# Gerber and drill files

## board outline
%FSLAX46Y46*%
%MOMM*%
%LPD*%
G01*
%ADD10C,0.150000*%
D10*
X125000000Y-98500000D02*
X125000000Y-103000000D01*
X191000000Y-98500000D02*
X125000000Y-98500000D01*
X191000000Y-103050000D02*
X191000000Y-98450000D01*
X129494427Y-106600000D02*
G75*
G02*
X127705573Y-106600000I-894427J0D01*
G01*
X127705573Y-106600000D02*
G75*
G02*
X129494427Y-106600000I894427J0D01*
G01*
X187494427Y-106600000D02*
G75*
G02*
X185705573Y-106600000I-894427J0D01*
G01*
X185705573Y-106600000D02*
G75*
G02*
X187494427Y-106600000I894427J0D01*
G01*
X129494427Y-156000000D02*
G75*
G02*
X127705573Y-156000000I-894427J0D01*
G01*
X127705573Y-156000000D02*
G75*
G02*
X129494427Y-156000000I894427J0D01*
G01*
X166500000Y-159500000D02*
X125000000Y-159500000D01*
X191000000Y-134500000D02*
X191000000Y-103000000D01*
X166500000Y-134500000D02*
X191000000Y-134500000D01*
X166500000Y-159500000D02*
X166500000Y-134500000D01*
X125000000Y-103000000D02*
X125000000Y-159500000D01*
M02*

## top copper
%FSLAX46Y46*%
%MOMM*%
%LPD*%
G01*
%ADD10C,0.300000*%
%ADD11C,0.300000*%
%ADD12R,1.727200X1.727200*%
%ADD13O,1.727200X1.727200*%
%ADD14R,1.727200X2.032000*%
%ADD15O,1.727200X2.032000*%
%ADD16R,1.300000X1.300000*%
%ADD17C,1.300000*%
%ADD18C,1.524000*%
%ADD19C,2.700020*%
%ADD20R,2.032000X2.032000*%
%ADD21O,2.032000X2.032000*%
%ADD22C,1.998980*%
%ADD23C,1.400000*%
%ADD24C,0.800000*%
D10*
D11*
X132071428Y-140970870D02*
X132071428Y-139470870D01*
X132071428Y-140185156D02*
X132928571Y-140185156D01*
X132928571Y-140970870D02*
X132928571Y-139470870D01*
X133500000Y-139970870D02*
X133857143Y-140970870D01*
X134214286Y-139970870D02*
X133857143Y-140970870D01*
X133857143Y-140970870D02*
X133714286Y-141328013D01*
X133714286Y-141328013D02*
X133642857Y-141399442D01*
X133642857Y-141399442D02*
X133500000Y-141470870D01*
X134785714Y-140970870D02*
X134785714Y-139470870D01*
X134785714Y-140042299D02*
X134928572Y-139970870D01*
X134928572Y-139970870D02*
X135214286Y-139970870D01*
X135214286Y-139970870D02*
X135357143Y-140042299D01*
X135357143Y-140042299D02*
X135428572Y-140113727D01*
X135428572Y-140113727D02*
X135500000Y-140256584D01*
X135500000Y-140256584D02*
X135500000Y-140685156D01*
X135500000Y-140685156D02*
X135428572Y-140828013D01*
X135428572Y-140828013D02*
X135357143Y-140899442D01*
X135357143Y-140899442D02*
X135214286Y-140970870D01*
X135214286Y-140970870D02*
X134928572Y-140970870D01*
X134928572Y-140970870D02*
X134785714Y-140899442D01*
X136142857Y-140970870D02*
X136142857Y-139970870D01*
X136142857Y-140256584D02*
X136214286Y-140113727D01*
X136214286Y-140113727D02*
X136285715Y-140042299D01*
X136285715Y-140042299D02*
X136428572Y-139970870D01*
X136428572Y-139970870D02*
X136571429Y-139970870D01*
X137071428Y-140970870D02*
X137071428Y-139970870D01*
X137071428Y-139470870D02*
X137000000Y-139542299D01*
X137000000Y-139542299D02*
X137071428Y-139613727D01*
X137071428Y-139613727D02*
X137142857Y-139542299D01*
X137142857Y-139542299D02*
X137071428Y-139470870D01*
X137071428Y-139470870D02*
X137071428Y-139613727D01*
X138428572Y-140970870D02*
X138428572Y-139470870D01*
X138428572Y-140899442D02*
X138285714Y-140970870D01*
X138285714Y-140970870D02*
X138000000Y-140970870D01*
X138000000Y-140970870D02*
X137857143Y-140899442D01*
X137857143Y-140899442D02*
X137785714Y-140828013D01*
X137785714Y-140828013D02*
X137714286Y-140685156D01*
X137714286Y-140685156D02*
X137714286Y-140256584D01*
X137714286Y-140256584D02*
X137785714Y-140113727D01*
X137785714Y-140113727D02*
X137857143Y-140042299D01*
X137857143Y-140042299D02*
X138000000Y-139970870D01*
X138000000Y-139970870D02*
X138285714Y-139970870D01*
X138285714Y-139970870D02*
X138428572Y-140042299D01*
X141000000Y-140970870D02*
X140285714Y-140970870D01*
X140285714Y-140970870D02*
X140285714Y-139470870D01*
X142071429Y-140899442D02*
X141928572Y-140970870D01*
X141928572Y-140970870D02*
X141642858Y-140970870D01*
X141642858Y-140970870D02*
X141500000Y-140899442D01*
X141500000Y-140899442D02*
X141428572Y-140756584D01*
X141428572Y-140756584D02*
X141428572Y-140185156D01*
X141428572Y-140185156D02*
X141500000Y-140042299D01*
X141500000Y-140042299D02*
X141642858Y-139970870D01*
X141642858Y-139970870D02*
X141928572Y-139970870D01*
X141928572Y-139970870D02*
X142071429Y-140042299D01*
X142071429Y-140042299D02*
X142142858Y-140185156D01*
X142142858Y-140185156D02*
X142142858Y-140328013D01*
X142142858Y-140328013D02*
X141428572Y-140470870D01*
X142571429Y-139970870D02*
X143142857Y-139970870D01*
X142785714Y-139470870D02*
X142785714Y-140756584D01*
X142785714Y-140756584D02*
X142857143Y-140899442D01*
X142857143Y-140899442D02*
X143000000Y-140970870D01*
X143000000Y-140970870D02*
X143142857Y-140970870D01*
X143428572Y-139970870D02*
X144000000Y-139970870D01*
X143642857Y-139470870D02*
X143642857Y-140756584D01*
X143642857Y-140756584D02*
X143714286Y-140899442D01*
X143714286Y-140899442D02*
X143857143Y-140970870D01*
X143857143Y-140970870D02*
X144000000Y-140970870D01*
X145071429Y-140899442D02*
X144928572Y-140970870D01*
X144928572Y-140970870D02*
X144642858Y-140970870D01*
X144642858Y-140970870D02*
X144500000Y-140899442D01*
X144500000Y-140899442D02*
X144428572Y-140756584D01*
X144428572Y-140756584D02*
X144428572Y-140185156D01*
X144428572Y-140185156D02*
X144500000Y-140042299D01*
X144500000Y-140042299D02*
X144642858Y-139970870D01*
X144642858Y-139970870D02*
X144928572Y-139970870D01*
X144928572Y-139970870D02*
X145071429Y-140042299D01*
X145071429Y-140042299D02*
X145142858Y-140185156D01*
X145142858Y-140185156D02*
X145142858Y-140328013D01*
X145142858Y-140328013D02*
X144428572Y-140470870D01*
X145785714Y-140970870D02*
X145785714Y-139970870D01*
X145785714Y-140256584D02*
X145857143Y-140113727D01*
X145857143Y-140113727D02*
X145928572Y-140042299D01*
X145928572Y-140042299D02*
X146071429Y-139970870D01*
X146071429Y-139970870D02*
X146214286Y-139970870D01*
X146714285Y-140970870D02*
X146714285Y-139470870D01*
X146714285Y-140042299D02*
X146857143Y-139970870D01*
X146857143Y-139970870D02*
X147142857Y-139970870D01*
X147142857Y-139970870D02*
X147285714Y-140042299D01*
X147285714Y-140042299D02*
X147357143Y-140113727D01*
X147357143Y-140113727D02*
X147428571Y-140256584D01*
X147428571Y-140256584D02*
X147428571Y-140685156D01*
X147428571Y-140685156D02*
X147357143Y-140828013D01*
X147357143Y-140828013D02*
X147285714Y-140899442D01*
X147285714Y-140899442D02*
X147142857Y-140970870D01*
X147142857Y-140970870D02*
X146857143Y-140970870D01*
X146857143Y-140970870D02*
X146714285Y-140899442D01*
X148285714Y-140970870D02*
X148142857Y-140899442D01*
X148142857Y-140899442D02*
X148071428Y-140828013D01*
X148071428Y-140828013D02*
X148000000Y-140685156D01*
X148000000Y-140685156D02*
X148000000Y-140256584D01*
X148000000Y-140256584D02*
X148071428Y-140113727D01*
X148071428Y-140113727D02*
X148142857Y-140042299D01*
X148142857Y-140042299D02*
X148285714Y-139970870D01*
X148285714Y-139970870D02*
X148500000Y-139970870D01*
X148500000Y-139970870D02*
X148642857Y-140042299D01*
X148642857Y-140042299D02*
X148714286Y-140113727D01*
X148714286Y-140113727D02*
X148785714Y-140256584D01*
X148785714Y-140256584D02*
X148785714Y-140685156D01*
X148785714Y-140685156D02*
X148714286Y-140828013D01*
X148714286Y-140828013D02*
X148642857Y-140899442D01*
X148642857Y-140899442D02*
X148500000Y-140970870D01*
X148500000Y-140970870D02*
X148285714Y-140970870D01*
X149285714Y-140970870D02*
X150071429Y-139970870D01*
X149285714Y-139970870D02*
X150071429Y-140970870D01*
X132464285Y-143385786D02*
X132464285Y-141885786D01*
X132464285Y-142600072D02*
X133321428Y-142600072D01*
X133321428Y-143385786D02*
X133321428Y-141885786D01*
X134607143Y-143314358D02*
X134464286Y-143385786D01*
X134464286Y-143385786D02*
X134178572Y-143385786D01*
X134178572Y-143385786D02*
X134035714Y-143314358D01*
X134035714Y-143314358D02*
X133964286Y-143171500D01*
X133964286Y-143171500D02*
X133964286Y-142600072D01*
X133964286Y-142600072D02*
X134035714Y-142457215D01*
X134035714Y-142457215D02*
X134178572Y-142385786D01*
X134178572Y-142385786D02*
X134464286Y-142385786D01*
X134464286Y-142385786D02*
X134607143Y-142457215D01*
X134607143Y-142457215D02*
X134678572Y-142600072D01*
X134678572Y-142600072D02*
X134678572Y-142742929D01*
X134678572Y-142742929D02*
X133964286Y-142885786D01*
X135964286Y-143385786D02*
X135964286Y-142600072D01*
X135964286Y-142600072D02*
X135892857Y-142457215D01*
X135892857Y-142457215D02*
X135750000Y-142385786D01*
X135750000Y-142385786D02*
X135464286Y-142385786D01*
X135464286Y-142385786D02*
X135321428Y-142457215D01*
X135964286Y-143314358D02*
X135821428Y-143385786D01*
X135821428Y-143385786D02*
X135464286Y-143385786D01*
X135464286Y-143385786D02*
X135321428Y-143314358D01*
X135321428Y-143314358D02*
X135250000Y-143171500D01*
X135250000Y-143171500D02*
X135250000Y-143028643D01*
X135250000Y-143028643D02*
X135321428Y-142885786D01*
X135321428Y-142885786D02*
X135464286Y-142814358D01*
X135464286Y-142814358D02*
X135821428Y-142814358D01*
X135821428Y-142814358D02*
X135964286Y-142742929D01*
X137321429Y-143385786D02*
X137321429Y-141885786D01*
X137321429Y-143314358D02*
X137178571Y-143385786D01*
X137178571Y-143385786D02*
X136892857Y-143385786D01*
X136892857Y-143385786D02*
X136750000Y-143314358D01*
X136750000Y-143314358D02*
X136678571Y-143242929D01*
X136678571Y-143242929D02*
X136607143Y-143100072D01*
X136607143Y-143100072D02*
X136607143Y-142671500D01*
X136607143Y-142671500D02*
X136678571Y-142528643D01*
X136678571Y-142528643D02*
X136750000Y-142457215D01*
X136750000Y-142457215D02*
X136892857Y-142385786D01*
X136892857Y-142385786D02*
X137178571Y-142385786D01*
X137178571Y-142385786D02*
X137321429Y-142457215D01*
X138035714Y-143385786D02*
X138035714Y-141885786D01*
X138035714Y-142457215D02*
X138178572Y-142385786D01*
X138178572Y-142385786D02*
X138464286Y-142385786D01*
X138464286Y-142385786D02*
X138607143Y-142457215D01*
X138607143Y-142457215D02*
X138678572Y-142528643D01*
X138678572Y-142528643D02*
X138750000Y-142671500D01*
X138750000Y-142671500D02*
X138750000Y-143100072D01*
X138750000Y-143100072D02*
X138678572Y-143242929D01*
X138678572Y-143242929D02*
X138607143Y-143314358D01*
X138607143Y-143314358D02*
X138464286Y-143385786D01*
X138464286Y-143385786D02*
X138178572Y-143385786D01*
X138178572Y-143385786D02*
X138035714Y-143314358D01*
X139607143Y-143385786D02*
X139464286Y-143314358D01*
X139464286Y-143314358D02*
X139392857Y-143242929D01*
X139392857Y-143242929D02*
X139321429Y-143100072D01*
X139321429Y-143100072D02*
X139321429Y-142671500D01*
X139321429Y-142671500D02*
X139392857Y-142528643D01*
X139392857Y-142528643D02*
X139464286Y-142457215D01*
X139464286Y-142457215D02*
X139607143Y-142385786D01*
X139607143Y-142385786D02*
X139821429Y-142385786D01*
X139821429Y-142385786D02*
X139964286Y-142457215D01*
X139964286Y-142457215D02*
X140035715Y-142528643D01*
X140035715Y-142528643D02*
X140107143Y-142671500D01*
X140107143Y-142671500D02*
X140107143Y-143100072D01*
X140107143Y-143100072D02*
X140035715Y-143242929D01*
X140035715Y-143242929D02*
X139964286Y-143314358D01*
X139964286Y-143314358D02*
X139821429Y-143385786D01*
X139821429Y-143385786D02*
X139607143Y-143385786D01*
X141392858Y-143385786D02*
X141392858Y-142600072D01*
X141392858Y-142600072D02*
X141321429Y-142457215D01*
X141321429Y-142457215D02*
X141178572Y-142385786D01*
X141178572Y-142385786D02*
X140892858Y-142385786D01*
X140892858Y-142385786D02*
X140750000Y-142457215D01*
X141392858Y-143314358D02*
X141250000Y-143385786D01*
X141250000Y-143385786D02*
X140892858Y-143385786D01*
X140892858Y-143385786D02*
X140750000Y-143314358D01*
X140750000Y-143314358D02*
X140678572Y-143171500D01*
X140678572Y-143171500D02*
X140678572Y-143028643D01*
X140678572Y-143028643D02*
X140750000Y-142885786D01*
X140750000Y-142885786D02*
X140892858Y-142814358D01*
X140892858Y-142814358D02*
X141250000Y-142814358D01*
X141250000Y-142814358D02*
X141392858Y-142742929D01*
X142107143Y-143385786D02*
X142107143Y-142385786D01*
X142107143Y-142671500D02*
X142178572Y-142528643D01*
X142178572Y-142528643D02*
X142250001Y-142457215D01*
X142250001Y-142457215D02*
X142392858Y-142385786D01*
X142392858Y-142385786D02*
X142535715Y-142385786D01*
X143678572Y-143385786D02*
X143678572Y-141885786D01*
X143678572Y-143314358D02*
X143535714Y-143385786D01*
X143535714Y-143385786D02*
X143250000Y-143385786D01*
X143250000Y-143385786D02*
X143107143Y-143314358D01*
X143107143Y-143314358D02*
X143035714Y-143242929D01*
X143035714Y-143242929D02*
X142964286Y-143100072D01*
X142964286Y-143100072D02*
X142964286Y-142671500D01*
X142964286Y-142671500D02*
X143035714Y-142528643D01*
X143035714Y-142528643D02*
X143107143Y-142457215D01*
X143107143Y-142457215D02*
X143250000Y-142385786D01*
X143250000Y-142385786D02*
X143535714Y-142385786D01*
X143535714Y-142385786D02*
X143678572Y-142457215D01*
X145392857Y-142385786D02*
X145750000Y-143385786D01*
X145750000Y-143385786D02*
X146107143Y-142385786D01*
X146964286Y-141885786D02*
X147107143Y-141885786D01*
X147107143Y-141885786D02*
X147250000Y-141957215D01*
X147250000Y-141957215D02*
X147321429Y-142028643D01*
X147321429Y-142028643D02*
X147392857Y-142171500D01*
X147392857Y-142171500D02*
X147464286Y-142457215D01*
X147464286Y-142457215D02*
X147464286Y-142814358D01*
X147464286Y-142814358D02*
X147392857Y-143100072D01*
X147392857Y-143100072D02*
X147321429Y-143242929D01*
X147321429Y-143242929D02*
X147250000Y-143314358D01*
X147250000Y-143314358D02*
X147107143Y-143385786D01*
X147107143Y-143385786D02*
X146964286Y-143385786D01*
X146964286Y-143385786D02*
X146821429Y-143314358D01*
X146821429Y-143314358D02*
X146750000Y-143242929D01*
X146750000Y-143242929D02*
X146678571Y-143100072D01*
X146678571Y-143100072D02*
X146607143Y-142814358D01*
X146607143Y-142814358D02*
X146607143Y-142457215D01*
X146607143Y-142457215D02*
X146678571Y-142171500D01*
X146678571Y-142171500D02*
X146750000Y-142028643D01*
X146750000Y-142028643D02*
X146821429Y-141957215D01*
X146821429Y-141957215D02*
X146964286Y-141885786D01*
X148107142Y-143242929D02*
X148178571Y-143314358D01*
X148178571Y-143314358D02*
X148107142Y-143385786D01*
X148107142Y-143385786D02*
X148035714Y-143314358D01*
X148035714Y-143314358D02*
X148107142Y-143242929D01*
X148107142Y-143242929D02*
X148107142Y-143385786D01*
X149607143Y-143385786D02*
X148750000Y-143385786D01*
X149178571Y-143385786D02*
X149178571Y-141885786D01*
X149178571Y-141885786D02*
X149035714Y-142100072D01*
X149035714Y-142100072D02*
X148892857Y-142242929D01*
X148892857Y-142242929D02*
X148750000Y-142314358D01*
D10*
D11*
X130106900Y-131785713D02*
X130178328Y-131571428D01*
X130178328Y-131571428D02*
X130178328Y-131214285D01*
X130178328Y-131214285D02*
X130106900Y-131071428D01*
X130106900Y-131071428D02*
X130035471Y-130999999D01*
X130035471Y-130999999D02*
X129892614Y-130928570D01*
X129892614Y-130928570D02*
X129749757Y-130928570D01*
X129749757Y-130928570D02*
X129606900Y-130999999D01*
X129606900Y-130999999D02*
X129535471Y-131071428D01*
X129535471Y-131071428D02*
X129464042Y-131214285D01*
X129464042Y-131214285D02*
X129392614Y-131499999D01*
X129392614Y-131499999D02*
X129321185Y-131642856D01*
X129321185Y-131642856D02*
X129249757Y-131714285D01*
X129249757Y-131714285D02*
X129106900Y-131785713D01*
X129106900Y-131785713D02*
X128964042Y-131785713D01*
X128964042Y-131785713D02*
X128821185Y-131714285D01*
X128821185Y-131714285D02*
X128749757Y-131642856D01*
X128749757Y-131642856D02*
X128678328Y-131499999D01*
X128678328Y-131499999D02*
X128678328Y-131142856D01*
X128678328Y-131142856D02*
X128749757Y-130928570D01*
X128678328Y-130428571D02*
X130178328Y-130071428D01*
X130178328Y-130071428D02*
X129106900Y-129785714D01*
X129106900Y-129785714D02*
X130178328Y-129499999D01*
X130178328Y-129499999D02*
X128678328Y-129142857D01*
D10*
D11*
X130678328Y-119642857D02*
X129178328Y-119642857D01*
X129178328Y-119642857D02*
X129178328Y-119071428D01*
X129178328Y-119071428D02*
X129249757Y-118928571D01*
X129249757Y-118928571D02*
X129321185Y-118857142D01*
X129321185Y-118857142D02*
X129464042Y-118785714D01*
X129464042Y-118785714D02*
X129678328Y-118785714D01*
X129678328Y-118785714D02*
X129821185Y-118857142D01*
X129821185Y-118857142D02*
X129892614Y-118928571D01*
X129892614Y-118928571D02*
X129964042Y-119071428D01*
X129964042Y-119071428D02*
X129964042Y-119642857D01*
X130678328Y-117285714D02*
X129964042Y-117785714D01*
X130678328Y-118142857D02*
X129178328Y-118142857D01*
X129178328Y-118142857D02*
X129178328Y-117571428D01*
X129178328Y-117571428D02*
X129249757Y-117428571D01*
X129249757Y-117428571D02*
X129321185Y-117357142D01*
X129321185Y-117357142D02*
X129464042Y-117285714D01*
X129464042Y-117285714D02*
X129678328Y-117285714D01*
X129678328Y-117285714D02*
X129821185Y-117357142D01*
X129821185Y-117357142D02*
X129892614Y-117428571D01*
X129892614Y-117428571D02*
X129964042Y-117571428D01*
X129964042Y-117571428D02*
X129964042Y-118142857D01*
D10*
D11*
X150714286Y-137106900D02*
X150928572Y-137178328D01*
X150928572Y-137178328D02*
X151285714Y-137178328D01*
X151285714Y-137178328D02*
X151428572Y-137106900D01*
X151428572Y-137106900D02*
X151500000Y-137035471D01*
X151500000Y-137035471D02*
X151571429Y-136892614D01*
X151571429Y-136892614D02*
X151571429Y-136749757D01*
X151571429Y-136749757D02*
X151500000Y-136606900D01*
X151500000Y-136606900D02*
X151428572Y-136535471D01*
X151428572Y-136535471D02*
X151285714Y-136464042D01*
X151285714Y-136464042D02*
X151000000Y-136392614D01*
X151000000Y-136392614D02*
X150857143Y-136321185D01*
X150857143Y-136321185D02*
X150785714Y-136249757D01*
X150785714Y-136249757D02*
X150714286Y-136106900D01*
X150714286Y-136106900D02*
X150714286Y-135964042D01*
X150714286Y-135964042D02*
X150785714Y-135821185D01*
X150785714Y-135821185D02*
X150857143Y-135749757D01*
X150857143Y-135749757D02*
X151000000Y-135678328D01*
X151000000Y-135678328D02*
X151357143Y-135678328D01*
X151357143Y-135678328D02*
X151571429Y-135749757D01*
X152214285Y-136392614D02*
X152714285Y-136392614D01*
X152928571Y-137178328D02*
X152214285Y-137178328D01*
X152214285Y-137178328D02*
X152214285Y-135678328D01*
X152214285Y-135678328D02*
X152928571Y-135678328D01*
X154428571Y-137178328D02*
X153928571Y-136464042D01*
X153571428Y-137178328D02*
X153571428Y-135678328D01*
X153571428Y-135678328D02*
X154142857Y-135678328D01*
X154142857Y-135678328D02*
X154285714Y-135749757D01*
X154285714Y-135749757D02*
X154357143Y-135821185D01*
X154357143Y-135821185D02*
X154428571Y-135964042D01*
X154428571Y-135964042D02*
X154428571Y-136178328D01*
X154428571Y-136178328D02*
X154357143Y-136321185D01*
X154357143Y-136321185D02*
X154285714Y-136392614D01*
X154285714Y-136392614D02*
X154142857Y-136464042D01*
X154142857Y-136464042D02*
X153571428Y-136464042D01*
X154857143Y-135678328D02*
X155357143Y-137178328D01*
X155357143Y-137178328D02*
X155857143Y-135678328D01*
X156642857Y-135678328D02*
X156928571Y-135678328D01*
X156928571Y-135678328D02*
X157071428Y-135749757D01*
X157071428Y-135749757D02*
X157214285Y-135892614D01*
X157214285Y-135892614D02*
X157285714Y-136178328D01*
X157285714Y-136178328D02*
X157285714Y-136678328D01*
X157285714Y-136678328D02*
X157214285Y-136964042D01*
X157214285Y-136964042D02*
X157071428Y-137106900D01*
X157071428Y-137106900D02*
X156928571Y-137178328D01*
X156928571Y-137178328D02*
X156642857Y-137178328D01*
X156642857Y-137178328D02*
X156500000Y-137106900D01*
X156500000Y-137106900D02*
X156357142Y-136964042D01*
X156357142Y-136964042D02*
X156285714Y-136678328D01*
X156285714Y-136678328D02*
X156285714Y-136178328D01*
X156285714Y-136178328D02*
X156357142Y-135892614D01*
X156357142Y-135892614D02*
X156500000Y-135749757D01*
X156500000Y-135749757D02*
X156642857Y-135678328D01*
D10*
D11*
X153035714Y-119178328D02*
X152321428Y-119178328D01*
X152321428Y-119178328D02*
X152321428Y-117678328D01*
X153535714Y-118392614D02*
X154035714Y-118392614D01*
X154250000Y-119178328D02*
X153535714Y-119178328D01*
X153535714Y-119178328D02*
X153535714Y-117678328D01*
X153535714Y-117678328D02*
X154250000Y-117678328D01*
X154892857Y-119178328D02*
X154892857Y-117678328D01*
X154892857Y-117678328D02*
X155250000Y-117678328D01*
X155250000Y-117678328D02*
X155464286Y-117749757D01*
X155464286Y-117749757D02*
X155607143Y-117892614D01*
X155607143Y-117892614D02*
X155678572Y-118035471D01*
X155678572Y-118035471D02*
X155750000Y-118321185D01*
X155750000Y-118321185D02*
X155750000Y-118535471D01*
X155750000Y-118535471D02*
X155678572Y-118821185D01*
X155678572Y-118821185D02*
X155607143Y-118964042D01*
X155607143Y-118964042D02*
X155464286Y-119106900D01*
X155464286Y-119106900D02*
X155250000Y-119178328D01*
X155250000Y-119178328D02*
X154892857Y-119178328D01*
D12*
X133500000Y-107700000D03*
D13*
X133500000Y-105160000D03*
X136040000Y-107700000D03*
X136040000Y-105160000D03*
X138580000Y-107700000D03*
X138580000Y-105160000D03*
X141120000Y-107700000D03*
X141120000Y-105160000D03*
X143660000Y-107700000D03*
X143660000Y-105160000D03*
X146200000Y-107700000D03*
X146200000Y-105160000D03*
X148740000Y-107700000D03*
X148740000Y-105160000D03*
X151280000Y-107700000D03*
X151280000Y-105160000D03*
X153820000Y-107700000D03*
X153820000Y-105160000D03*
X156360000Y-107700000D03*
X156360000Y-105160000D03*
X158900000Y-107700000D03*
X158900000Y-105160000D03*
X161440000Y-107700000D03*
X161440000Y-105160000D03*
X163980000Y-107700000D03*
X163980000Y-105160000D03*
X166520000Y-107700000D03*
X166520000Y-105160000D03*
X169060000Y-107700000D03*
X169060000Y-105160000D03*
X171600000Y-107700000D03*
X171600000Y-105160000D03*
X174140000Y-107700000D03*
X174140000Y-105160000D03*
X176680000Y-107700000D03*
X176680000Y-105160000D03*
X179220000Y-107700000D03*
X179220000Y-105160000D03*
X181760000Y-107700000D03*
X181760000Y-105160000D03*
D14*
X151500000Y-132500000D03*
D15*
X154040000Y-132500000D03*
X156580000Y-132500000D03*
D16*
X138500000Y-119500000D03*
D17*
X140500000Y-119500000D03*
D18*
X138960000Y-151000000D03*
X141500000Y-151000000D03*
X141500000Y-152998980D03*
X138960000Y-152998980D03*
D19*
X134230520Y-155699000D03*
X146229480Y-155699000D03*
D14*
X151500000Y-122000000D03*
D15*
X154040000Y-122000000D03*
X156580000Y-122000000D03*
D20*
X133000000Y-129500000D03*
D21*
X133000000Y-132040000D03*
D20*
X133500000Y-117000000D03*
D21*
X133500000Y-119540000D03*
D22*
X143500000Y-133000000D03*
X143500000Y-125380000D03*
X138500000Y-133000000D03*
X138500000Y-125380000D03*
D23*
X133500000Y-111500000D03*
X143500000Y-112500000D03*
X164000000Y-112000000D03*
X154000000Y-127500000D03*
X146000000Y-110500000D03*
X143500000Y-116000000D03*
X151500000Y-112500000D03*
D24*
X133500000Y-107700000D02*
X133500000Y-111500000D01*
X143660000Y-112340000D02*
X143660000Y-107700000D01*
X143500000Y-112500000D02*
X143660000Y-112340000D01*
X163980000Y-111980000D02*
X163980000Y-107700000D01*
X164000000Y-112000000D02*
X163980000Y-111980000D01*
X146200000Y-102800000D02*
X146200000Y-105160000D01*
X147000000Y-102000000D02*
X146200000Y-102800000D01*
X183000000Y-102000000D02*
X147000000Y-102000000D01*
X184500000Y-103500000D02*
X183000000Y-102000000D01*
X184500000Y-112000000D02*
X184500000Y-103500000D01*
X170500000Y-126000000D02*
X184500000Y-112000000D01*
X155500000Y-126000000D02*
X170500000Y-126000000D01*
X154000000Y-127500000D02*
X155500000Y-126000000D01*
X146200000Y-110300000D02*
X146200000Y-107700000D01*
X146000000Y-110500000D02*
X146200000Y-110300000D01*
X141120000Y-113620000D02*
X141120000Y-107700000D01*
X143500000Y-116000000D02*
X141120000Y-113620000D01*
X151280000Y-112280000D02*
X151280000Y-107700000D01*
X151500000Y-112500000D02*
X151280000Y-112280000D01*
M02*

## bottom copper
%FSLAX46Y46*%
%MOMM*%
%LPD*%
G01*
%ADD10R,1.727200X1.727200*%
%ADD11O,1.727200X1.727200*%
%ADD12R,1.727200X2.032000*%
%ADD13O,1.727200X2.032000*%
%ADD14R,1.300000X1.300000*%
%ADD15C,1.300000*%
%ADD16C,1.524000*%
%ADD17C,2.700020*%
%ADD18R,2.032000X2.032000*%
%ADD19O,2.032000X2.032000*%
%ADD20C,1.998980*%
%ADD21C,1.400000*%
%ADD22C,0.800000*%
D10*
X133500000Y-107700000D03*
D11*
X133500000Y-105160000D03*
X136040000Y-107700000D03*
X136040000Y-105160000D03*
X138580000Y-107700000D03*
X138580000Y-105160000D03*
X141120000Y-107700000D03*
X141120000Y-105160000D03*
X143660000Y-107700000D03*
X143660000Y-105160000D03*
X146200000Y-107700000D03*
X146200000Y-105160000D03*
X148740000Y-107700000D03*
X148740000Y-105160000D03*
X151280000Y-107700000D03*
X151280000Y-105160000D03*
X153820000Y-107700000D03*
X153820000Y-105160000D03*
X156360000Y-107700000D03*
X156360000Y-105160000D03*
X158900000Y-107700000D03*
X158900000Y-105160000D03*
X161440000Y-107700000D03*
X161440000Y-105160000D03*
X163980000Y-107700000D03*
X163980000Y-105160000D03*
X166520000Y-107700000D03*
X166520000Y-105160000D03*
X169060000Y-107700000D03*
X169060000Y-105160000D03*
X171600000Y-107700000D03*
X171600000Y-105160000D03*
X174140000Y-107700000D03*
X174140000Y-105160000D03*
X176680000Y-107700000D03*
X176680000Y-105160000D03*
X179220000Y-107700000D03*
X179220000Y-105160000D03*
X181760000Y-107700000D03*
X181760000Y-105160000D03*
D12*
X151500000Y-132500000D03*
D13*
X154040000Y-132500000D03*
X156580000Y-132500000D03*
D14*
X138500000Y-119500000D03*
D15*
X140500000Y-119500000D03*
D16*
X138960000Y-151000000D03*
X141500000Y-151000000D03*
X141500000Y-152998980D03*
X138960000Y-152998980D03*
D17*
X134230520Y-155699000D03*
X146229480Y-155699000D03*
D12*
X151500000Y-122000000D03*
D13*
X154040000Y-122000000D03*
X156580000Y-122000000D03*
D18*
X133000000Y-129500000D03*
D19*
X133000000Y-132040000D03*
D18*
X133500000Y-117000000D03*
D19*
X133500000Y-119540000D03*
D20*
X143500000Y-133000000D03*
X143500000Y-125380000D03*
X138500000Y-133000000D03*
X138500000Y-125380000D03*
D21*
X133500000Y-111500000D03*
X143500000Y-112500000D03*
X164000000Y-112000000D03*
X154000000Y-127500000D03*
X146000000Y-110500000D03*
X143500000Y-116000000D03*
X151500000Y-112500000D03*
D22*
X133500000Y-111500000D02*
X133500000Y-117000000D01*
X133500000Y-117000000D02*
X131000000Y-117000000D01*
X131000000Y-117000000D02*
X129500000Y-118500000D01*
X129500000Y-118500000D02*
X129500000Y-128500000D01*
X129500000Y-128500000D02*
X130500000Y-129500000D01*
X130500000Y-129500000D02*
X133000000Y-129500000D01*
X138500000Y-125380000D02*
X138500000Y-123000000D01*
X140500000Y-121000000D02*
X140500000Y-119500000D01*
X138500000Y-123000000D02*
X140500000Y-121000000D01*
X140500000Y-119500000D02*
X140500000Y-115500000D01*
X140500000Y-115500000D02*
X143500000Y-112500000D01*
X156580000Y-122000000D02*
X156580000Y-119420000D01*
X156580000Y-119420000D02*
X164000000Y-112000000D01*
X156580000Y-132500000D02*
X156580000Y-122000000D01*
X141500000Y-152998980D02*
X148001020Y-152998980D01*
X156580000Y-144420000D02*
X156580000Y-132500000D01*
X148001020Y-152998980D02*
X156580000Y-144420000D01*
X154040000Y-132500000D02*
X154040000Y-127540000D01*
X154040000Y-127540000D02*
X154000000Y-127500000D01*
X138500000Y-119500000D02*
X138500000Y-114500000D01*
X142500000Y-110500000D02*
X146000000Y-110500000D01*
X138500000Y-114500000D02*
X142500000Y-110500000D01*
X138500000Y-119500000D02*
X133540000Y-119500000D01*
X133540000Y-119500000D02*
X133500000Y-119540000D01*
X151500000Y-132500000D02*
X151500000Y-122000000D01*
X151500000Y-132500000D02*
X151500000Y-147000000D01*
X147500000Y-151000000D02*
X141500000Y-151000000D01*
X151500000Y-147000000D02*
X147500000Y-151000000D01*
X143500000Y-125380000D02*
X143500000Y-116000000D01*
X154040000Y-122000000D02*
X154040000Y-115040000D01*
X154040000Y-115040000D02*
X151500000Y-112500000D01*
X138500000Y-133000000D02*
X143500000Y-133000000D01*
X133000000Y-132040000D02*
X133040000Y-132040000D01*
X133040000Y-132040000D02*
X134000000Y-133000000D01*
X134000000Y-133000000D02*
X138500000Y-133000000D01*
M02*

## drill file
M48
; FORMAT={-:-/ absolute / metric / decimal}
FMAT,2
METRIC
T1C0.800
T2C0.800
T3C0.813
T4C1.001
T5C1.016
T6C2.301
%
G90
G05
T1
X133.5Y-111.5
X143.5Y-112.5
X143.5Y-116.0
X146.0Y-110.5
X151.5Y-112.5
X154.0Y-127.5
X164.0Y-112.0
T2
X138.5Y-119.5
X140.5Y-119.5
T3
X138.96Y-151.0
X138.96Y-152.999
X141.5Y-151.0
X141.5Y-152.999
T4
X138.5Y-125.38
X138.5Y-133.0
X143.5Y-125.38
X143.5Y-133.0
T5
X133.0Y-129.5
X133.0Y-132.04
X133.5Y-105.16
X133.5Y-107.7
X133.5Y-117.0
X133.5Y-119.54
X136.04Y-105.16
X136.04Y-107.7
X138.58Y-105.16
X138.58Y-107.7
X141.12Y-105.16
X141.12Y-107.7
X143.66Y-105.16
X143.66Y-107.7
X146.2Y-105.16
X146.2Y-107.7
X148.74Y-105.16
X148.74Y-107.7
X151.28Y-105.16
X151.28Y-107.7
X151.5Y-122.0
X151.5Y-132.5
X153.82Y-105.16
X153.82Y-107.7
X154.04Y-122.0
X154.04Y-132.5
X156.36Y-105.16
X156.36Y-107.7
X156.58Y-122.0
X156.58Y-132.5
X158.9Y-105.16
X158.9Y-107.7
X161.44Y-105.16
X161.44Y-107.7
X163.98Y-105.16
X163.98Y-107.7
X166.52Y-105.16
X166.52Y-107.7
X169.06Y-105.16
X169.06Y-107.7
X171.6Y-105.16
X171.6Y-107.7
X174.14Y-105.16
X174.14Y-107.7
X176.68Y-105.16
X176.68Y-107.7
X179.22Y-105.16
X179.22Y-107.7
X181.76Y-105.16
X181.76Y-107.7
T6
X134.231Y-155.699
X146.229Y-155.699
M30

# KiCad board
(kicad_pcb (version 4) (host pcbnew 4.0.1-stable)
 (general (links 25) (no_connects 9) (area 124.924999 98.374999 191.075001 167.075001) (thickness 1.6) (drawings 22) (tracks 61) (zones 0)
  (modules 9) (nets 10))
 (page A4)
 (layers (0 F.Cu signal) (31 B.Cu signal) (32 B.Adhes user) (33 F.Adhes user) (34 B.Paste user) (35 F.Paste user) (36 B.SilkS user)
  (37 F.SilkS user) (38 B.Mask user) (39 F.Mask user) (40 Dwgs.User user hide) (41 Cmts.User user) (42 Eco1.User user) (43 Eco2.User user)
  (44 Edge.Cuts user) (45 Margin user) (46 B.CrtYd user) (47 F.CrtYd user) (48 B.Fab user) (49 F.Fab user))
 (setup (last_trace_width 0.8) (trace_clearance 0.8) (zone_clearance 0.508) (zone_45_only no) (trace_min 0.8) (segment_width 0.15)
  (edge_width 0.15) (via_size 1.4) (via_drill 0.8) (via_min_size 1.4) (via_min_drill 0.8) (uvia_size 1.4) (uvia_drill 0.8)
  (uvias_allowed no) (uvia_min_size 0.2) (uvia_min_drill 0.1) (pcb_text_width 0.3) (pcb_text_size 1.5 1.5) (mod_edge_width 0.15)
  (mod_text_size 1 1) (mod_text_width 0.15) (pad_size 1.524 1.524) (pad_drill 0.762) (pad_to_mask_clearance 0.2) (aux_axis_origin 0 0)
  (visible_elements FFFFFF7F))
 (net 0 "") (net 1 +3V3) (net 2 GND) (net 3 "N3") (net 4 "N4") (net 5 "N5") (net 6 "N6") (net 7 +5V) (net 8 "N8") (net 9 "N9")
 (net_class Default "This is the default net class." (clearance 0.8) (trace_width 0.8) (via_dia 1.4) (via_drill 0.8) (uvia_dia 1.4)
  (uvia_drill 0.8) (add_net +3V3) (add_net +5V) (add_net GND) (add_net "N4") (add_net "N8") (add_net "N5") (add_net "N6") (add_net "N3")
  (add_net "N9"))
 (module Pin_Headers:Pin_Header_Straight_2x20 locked (layer F.Cu) (at 133.5 107.7 90)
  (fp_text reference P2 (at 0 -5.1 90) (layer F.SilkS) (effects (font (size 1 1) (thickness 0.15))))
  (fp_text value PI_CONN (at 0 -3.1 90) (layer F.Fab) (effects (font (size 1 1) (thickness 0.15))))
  (pad 1 thru_hole rect (at 0 0 90) (size 1.7272 1.7272) (drill 1.016) (layers *.Cu *.Mask F.SilkS) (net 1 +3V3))
  (pad 2 thru_hole oval (at 2.54 0 90) (size 1.7272 1.7272) (drill 1.016) (layers *.Cu *.Mask F.SilkS))
  (pad 3 thru_hole oval (at 0 2.54 90) (size 1.7272 1.7272) (drill 1.016) (layers *.Cu *.Mask F.SilkS))
  (pad 4 thru_hole oval (at 2.54 2.54 90) (size 1.7272 1.7272) (drill 1.016) (layers *.Cu *.Mask F.SilkS))
  (pad 5 thru_hole oval (at 0 5.08 90) (size 1.7272 1.7272) (drill 1.016) (layers *.Cu *.Mask F.SilkS))
  (pad 6 thru_hole oval (at 2.54 5.08 90) (size 1.7272 1.7272) (drill 1.016) (layers *.Cu *.Mask F.SilkS) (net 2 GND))
  (pad 7 thru_hole oval (at 0 7.62 90) (size 1.7272 1.7272) (drill 1.016) (layers *.Cu *.Mask F.SilkS) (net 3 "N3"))
  (pad 8 thru_hole oval (at 2.54 7.62 90) (size 1.7272 1.7272) (drill 1.016) (layers *.Cu *.Mask F.SilkS))
  (pad 9 thru_hole oval (at 0 10.16 90) (size 1.7272 1.7272) (drill 1.016) (layers *.Cu *.Mask F.SilkS) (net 2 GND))
  (pad 10 thru_hole oval (at 2.54 10.16 90) (size 1.7272 1.7272) (drill 1.016) (layers *.Cu *.Mask F.SilkS))
  (pad 11 thru_hole oval (at 0 12.7 90) (size 1.7272 1.7272) (drill 1.016) (layers *.Cu *.Mask F.SilkS) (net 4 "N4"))
  (pad 12 thru_hole oval (at 2.54 12.7 90) (size 1.7272 1.7272) (drill 1.016) (layers *.Cu *.Mask F.SilkS) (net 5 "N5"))
  (pad 13 thru_hole oval (at 0 15.24 90) (size 1.7272 1.7272) (drill 1.016) (layers *.Cu *.Mask F.SilkS))
  (pad 14 thru_hole oval (at 2.54 15.24 90) (size 1.7272 1.7272) (drill 1.016) (layers *.Cu *.Mask F.SilkS) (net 2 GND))
  (pad 15 thru_hole oval (at 0 17.78 90) (size 1.7272 1.7272) (drill 1.016) (layers *.Cu *.Mask F.SilkS) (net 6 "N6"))
  (pad 16 thru_hole oval (at 2.54 17.78 90) (size 1.7272 1.7272) (drill 1.016) (layers *.Cu *.Mask F.SilkS))
  (pad 17 thru_hole oval (at 0 20.32 90) (size 1.7272 1.7272) (drill 1.016) (layers *.Cu *.Mask F.SilkS) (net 1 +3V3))
  (pad 18 thru_hole oval (at 2.54 20.32 90) (size 1.7272 1.7272) (drill 1.016) (layers *.Cu *.Mask F.SilkS))
  (pad 19 thru_hole oval (at 0 22.86 90) (size 1.7272 1.7272) (drill 1.016) (layers *.Cu *.Mask F.SilkS))
  (pad 20 thru_hole oval (at 2.54 22.86 90) (size 1.7272 1.7272) (drill 1.016) (layers *.Cu *.Mask F.SilkS) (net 2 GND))
  (pad 21 thru_hole oval (at 0 25.4 90) (size 1.7272 1.7272) (drill 1.016) (layers *.Cu *.Mask F.SilkS))
  (pad 22 thru_hole oval (at 2.54 25.4 90) (size 1.7272 1.7272) (drill 1.016) (layers *.Cu *.Mask F.SilkS))
  (pad 23 thru_hole oval (at 0 27.94 90) (size 1.7272 1.7272) (drill 1.016) (layers *.Cu *.Mask F.SilkS))
  (pad 24 thru_hole oval (at 2.54 27.94 90) (size 1.7272 1.7272) (drill 1.016) (layers *.Cu *.Mask F.SilkS))
  (pad 25 thru_hole oval (at 0 30.48 90) (size 1.7272 1.7272) (drill 1.016) (layers *.Cu *.Mask F.SilkS) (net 2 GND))
  (pad 26 thru_hole oval (at 2.54 30.48 90) (size 1.7272 1.7272) (drill 1.016) (layers *.Cu *.Mask F.SilkS))
  (pad 27 thru_hole oval (at 0 33.02 90) (size 1.7272 1.7272) (drill 1.016) (layers *.Cu *.Mask F.SilkS))
  (pad 28 thru_hole oval (at 2.54 33.02 90) (size 1.7272 1.7272) (drill 1.016) (layers *.Cu *.Mask F.SilkS))
  (pad 29 thru_hole oval (at 0 35.56 90) (size 1.7272 1.7272) (drill 1.016) (layers *.Cu *.Mask F.SilkS))
  (pad 30 thru_hole oval (at 2.54 35.56 90) (size 1.7272 1.7272) (drill 1.016) (layers *.Cu *.Mask F.SilkS) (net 2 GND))
  (pad 31 thru_hole oval (at 0 38.1 90) (size 1.7272 1.7272) (drill 1.016) (layers *.Cu *.Mask F.SilkS))
  (pad 32 thru_hole oval (at 2.54 38.1 90) (size 1.7272 1.7272) (drill 1.016) (layers *.Cu *.Mask F.SilkS))
  (pad 33 thru_hole oval (at 0 40.64 90) (size 1.7272 1.7272) (drill 1.016) (layers *.Cu *.Mask F.SilkS))
  (pad 34 thru_hole oval (at 2.54 40.64 90) (size 1.7272 1.7272) (drill 1.016) (layers *.Cu *.Mask F.SilkS) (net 2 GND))
  (pad 35 thru_hole oval (at 0 43.18 90) (size 1.7272 1.7272) (drill 1.016) (layers *.Cu *.Mask F.SilkS))
  (pad 36 thru_hole oval (at 2.54 43.18 90) (size 1.7272 1.7272) (drill 1.016) (layers *.Cu *.Mask F.SilkS))
  (pad 37 thru_hole oval (at 0 45.72 90) (size 1.7272 1.7272) (drill 1.016) (layers *.Cu *.Mask F.SilkS))
  (pad 38 thru_hole oval (at 2.54 45.72 90) (size 1.7272 1.7272) (drill 1.016) (layers *.Cu *.Mask F.SilkS))
  (pad 39 thru_hole oval (at 0 48.26 90) (size 1.7272 1.7272) (drill 1.016) (layers *.Cu *.Mask F.SilkS) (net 2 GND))
  (pad 40 thru_hole oval (at 2.54 48.26 90) (size 1.7272 1.7272) (drill 1.016) (layers *.Cu *.Mask F.SilkS)))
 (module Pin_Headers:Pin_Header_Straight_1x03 (layer F.Cu) (at 151.5 132.5 90)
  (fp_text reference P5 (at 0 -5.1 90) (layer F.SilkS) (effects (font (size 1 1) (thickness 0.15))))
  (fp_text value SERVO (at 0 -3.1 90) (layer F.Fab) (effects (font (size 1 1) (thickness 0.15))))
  (pad 1 thru_hole rect (at 0 0 90) (size 2.032 1.7272) (drill 1.016) (layers *.Cu *.Mask F.SilkS) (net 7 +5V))
  (pad 2 thru_hole oval (at 0 2.54 90) (size 2.032 1.7272) (drill 1.016) (layers *.Cu *.Mask F.SilkS) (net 5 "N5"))
  (pad 3 thru_hole oval (at 0 5.08 90) (size 2.032 1.7272) (drill 1.016) (layers *.Cu *.Mask F.SilkS) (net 2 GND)))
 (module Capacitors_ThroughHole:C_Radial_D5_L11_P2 (layer F.Cu) (at 138.5 119.5)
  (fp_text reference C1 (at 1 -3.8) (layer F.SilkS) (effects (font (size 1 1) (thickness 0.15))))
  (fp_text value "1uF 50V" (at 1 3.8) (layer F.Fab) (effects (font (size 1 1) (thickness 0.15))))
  (pad 1 thru_hole rect (at 0 0) (size 1.3 1.3) (drill 0.8) (layers *.Cu *.Mask F.SilkS) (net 4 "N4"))
  (pad 2 thru_hole circle (at 2 0) (size 1.3 1.3) (drill 0.8) (layers *.Cu *.Mask F.SilkS) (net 2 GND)))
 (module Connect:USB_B (layer F.Cu) (at 141.5 151 270)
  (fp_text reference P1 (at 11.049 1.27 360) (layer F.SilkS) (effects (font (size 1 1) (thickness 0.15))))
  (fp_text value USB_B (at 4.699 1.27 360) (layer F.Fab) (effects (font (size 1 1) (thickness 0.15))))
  (pad 2 thru_hole circle (at 0 2.54 180) (size 1.524 1.524) (drill 0.8128) (layers *.Cu *.Mask F.SilkS))
  (pad 1 thru_hole circle (at 0 0 180) (size 1.524 1.524) (drill 0.8128) (layers *.Cu *.Mask F.SilkS) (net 7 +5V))
  (pad 4 thru_hole circle (at 1.99898 0 180) (size 1.524 1.524) (drill 0.8128) (layers *.Cu *.Mask F.SilkS) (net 2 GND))
  (pad 3 thru_hole circle (at 1.99898 2.54 180) (size 1.524 1.524) (drill 0.8128) (layers *.Cu *.Mask F.SilkS))
  (pad 5 thru_hole circle (at 4.699 7.26948 180) (size 2.70002 2.70002) (drill 2.30124) (layers *.Cu *.Mask F.SilkS) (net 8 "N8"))
  (pad 5 thru_hole circle (at 4.699 -4.72948 180) (size 2.70002 2.70002) (drill 2.30124) (layers *.Cu *.Mask F.SilkS) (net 8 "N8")))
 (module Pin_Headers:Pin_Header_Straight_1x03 (layer F.Cu) (at 151.5 122 90)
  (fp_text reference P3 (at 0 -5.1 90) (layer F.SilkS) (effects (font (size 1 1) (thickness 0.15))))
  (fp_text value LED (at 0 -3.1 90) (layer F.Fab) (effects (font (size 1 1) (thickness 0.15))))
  (pad 1 thru_hole rect (at 0 0 90) (size 2.032 1.7272) (drill 1.016) (layers *.Cu *.Mask F.SilkS) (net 7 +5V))
  (pad 2 thru_hole oval (at 0 2.54 90) (size 2.032 1.7272) (drill 1.016) (layers *.Cu *.Mask F.SilkS) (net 6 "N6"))
  (pad 3 thru_hole oval (at 0 5.08 90) (size 2.032 1.7272) (drill 1.016) (layers *.Cu *.Mask F.SilkS) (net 2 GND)))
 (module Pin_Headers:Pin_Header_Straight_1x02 (layer F.Cu) (at 133 129.5)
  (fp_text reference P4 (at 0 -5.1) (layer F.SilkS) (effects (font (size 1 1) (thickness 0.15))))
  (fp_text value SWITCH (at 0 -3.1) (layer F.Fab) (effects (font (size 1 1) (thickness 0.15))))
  (pad 1 thru_hole rect (at 0 0) (size 2.032 2.032) (drill 1.016) (layers *.Cu *.Mask F.SilkS) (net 1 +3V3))
  (pad 2 thru_hole oval (at 0 2.54) (size 2.032 2.032) (drill 1.016) (layers *.Cu *.Mask F.SilkS) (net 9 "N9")))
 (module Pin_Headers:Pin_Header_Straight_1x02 (layer F.Cu) (at 133.5 117)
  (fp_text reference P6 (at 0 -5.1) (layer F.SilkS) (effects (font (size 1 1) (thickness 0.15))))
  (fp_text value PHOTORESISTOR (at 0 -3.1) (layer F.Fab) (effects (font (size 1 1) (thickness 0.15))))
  (pad 1 thru_hole rect (at 0 0) (size 2.032 2.032) (drill 1.016) (layers *.Cu *.Mask F.SilkS) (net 1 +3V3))
  (pad 2 thru_hole oval (at 0 2.54) (size 2.032 2.032) (drill 1.016) (layers *.Cu *.Mask F.SilkS) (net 4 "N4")))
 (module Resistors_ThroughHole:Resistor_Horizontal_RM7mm (layer F.Cu) (at 143.5 133 90)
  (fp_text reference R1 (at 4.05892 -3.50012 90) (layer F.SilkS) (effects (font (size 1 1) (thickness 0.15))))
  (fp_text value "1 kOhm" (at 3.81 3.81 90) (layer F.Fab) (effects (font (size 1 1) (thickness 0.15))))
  (pad 1 thru_hole circle (at 0 0 90) (size 1.99898 1.99898) (drill 1.00076) (layers *.Cu *.SilkS *.Mask) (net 9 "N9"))
  (pad 2 thru_hole circle (at 7.62 0 90) (size 1.99898 1.99898) (drill 1.00076) (layers *.Cu *.SilkS *.Mask) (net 3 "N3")))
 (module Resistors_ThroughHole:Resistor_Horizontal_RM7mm (layer F.Cu) (at 138.5 133 90)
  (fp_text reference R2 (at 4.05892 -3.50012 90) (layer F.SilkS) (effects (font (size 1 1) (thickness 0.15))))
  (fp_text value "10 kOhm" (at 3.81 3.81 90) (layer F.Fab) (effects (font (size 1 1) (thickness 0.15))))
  (pad 1 thru_hole circle (at 0 0 90) (size 1.99898 1.99898) (drill 1.00076) (layers *.Cu *.SilkS *.Mask) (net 9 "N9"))
  (pad 2 thru_hole circle (at 7.62 0 90) (size 1.99898 1.99898) (drill 1.00076) (layers *.Cu *.SilkS *.Mask) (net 2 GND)))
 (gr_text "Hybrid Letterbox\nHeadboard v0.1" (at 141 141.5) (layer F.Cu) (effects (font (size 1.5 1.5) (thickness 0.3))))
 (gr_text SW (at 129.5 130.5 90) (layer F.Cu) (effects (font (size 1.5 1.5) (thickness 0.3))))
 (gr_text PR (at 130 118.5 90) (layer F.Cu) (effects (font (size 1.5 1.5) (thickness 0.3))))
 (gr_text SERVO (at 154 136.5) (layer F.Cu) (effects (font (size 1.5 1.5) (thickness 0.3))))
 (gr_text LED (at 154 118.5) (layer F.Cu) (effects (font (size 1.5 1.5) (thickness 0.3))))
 (gr_line (start 125 98.5) (end 125 103) (angle 90) (layer Edge.Cuts) (width 0.15))
 (gr_line (start 191 98.5) (end 125 98.5) (angle 90) (layer Edge.Cuts) (width 0.15))
 (gr_line (start 191 103.05) (end 191 98.45) (angle 90) (layer Edge.Cuts) (width 0.15))
 (gr_circle (center 128.6 106.6) (end 127.8 106.2) (layer Edge.Cuts) (width 0.15))
 (gr_circle (center 186.6 106.6) (end 185.8 106.2) (layer Edge.Cuts) (width 0.15))
 (gr_circle (center 128.6 156) (end 127.8 155.6) (layer Edge.Cuts) (width 0.15))
 (gr_line (start 166.5 159.5) (end 125 159.5) (angle 90) (layer Edge.Cuts) (width 0.15))
 (gr_line (start 191 134.5) (end 191 103) (angle 90) (layer Edge.Cuts) (width 0.15))
 (gr_line (start 166.5 134.5) (end 191 134.5) (angle 90) (layer Edge.Cuts) (width 0.15))
 (gr_line (start 166.5 159.5) (end 166.5 134.5) (angle 90) (layer Edge.Cuts) (width 0.15))
 (gr_line (start 125 103) (end 125 159.5) (angle 90) (layer Edge.Cuts) (width 0.15))
 (segment (start 133.5 107.7) (end 133.5 111.5) (width 0.8) (layer F.Cu) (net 1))
 (segment (start 133.5 111.5) (end 133.5 117) (width 0.8) (layer B.Cu) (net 1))
 (via (at 133.5 111.5) (size 1.4) (drill 0.8) (layers F.Cu B.Cu) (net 1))
 (segment (start 133.5 117) (end 131 117) (width 0.8) (layer B.Cu) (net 1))
 (segment (start 131 117) (end 129.5 118.5) (width 0.8) (layer B.Cu) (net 1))
 (segment (start 129.5 118.5) (end 129.5 128.5) (width 0.8) (layer B.Cu) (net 1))
 (segment (start 129.5 128.5) (end 130.5 129.5) (width 0.8) (layer B.Cu) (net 1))
 (segment (start 130.5 129.5) (end 133 129.5) (width 0.8) (layer B.Cu) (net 1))
 (segment (start 138.5 125.38) (end 138.5 123) (width 0.8) (layer B.Cu) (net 2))
 (segment (start 140.5 121) (end 140.5 119.5) (width 0.8) (layer B.Cu) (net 2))
 (segment (start 138.5 123) (end 140.5 121) (width 0.8) (layer B.Cu) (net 2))
 (segment (start 140.5 119.5) (end 140.5 115.5) (width 0.8) (layer B.Cu) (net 2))
 (segment (start 143.66 112.34) (end 143.66 107.7) (width 0.8) (layer F.Cu) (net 2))
 (segment (start 143.5 112.5) (end 143.66 112.34) (width 0.8) (layer F.Cu) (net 2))
 (via (at 143.5 112.5) (size 1.4) (drill 0.8) (layers F.Cu B.Cu) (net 2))
 (segment (start 140.5 115.5) (end 143.5 112.5) (width 0.8) (layer B.Cu) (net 2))
 (segment (start 156.58 122) (end 156.58 119.42) (width 0.8) (layer B.Cu) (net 2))
 (segment (start 163.98 111.98) (end 163.98 107.7) (width 0.8) (layer F.Cu) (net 2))
 (segment (start 164 112) (end 163.98 111.98) (width 0.8) (layer F.Cu) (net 2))
 (via (at 164 112) (size 1.4) (drill 0.8) (layers F.Cu B.Cu) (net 2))
 (segment (start 156.58 119.42) (end 164 112) (width 0.8) (layer B.Cu) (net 2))
 (segment (start 156.58 132.5) (end 156.58 122) (width 0.8) (layer B.Cu) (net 2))
 (segment (start 141.5 152.99898) (end 148.00102 152.99898) (width 0.8) (layer B.Cu) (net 2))
 (segment (start 156.58 144.42) (end 156.58 132.5) (width 0.8) (layer B.Cu) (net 2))
 (segment (start 148.00102 152.99898) (end 156.58 144.42) (width 0.8) (layer B.Cu) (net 2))
 (segment (start 154.04 132.5) (end 154.04 127.54) (width 0.8) (layer B.Cu) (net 5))
 (segment (start 146.2 102.8) (end 146.2 105.16) (width 0.8) (layer F.Cu) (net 5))
 (segment (start 147 102) (end 146.2 102.8) (width 0.8) (layer F.Cu) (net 5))
 (segment (start 183 102) (end 147 102) (width 0.8) (layer F.Cu) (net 5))
 (segment (start 184.5 103.5) (end 183 102) (width 0.8) (layer F.Cu) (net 5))
 (segment (start 184.5 112) (end 184.5 103.5) (width 0.8) (layer F.Cu) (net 5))
 (segment (start 170.5 126) (end 184.5 112) (width 0.8) (layer F.Cu) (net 5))
 (segment (start 155.5 126) (end 170.5 126) (width 0.8) (layer F.Cu) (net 5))
 (segment (start 154 127.5) (end 155.5 126) (width 0.8) (layer F.Cu) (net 5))
 (via (at 154 127.5) (size 1.4) (drill 0.8) (layers F.Cu B.Cu) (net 5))
 (segment (start 154.04 127.54) (end 154 127.5) (width 0.8) (layer B.Cu) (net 5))
 (segment (start 138.5 119.5) (end 138.5 114.5) (width 0.8) (layer B.Cu) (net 4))
 (segment (start 146.2 110.3) (end 146.2 107.7) (width 0.8) (layer F.Cu) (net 4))
 (segment (start 146 110.5) (end 146.2 110.3) (width 0.8) (layer F.Cu) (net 4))
 (via (at 146 110.5) (size 1.4) (drill 0.8) (layers F.Cu B.Cu) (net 4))
 (segment (start 142.5 110.5) (end 146 110.5) (width 0.8) (layer B.Cu) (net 4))
 (segment (start 138.5 114.5) (end 142.5 110.5) (width 0.8) (layer B.Cu) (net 4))
 (segment (start 138.5 119.5) (end 133.54 119.5) (width 0.8) (layer B.Cu) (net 4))
 (segment (start 133.54 119.5) (end 133.5 119.54) (width 0.8) (layer B.Cu) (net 4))
 (segment (start 151.5 132.5) (end 151.5 122) (width 0.8) (layer B.Cu) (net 7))
 (segment (start 151.5 132.5) (end 151.5 147) (width 0.8) (layer B.Cu) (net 7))
 (segment (start 147.5 151) (end 141.5 151) (width 0.8) (layer B.Cu) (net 7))
 (segment (start 151.5 147) (end 147.5 151) (width 0.8) (layer B.Cu) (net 7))
 (segment (start 143.5 125.38) (end 143.5 116) (width 0.8) (layer B.Cu) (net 3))
 (segment (start 141.12 113.62) (end 141.12 107.7) (width 0.8) (layer F.Cu) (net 3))
 (segment (start 143.5 116) (end 141.12 113.62) (width 0.8) (layer F.Cu) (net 3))
 (via (at 143.5 116) (size 1.4) (drill 0.8) (layers F.Cu B.Cu) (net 3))
 (segment (start 154.04 122) (end 154.04 115.04) (width 0.8) (layer B.Cu) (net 6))
 (segment (start 151.28 112.28) (end 151.28 107.7) (width 0.8) (layer F.Cu) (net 6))
 (segment (start 151.5 112.5) (end 151.28 112.28) (width 0.8) (layer F.Cu) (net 6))
 (via (at 151.5 112.5) (size 1.4) (drill 0.8) (layers F.Cu B.Cu) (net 6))
 (segment (start 154.04 115.04) (end 151.5 112.5) (width 0.8) (layer B.Cu) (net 6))
 (segment (start 138.5 133) (end 143.5 133) (width 0.8) (layer B.Cu) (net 9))
 (segment (start 133 132.04) (end 133.04 132.04) (width 0.8) (layer B.Cu) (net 9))
 (segment (start 133.04 132.04) (end 134 133) (width 0.8) (layer B.Cu) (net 9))
 (segment (start 134 133) (end 138.5 133) (width 0.8) (layer B.Cu) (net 9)))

